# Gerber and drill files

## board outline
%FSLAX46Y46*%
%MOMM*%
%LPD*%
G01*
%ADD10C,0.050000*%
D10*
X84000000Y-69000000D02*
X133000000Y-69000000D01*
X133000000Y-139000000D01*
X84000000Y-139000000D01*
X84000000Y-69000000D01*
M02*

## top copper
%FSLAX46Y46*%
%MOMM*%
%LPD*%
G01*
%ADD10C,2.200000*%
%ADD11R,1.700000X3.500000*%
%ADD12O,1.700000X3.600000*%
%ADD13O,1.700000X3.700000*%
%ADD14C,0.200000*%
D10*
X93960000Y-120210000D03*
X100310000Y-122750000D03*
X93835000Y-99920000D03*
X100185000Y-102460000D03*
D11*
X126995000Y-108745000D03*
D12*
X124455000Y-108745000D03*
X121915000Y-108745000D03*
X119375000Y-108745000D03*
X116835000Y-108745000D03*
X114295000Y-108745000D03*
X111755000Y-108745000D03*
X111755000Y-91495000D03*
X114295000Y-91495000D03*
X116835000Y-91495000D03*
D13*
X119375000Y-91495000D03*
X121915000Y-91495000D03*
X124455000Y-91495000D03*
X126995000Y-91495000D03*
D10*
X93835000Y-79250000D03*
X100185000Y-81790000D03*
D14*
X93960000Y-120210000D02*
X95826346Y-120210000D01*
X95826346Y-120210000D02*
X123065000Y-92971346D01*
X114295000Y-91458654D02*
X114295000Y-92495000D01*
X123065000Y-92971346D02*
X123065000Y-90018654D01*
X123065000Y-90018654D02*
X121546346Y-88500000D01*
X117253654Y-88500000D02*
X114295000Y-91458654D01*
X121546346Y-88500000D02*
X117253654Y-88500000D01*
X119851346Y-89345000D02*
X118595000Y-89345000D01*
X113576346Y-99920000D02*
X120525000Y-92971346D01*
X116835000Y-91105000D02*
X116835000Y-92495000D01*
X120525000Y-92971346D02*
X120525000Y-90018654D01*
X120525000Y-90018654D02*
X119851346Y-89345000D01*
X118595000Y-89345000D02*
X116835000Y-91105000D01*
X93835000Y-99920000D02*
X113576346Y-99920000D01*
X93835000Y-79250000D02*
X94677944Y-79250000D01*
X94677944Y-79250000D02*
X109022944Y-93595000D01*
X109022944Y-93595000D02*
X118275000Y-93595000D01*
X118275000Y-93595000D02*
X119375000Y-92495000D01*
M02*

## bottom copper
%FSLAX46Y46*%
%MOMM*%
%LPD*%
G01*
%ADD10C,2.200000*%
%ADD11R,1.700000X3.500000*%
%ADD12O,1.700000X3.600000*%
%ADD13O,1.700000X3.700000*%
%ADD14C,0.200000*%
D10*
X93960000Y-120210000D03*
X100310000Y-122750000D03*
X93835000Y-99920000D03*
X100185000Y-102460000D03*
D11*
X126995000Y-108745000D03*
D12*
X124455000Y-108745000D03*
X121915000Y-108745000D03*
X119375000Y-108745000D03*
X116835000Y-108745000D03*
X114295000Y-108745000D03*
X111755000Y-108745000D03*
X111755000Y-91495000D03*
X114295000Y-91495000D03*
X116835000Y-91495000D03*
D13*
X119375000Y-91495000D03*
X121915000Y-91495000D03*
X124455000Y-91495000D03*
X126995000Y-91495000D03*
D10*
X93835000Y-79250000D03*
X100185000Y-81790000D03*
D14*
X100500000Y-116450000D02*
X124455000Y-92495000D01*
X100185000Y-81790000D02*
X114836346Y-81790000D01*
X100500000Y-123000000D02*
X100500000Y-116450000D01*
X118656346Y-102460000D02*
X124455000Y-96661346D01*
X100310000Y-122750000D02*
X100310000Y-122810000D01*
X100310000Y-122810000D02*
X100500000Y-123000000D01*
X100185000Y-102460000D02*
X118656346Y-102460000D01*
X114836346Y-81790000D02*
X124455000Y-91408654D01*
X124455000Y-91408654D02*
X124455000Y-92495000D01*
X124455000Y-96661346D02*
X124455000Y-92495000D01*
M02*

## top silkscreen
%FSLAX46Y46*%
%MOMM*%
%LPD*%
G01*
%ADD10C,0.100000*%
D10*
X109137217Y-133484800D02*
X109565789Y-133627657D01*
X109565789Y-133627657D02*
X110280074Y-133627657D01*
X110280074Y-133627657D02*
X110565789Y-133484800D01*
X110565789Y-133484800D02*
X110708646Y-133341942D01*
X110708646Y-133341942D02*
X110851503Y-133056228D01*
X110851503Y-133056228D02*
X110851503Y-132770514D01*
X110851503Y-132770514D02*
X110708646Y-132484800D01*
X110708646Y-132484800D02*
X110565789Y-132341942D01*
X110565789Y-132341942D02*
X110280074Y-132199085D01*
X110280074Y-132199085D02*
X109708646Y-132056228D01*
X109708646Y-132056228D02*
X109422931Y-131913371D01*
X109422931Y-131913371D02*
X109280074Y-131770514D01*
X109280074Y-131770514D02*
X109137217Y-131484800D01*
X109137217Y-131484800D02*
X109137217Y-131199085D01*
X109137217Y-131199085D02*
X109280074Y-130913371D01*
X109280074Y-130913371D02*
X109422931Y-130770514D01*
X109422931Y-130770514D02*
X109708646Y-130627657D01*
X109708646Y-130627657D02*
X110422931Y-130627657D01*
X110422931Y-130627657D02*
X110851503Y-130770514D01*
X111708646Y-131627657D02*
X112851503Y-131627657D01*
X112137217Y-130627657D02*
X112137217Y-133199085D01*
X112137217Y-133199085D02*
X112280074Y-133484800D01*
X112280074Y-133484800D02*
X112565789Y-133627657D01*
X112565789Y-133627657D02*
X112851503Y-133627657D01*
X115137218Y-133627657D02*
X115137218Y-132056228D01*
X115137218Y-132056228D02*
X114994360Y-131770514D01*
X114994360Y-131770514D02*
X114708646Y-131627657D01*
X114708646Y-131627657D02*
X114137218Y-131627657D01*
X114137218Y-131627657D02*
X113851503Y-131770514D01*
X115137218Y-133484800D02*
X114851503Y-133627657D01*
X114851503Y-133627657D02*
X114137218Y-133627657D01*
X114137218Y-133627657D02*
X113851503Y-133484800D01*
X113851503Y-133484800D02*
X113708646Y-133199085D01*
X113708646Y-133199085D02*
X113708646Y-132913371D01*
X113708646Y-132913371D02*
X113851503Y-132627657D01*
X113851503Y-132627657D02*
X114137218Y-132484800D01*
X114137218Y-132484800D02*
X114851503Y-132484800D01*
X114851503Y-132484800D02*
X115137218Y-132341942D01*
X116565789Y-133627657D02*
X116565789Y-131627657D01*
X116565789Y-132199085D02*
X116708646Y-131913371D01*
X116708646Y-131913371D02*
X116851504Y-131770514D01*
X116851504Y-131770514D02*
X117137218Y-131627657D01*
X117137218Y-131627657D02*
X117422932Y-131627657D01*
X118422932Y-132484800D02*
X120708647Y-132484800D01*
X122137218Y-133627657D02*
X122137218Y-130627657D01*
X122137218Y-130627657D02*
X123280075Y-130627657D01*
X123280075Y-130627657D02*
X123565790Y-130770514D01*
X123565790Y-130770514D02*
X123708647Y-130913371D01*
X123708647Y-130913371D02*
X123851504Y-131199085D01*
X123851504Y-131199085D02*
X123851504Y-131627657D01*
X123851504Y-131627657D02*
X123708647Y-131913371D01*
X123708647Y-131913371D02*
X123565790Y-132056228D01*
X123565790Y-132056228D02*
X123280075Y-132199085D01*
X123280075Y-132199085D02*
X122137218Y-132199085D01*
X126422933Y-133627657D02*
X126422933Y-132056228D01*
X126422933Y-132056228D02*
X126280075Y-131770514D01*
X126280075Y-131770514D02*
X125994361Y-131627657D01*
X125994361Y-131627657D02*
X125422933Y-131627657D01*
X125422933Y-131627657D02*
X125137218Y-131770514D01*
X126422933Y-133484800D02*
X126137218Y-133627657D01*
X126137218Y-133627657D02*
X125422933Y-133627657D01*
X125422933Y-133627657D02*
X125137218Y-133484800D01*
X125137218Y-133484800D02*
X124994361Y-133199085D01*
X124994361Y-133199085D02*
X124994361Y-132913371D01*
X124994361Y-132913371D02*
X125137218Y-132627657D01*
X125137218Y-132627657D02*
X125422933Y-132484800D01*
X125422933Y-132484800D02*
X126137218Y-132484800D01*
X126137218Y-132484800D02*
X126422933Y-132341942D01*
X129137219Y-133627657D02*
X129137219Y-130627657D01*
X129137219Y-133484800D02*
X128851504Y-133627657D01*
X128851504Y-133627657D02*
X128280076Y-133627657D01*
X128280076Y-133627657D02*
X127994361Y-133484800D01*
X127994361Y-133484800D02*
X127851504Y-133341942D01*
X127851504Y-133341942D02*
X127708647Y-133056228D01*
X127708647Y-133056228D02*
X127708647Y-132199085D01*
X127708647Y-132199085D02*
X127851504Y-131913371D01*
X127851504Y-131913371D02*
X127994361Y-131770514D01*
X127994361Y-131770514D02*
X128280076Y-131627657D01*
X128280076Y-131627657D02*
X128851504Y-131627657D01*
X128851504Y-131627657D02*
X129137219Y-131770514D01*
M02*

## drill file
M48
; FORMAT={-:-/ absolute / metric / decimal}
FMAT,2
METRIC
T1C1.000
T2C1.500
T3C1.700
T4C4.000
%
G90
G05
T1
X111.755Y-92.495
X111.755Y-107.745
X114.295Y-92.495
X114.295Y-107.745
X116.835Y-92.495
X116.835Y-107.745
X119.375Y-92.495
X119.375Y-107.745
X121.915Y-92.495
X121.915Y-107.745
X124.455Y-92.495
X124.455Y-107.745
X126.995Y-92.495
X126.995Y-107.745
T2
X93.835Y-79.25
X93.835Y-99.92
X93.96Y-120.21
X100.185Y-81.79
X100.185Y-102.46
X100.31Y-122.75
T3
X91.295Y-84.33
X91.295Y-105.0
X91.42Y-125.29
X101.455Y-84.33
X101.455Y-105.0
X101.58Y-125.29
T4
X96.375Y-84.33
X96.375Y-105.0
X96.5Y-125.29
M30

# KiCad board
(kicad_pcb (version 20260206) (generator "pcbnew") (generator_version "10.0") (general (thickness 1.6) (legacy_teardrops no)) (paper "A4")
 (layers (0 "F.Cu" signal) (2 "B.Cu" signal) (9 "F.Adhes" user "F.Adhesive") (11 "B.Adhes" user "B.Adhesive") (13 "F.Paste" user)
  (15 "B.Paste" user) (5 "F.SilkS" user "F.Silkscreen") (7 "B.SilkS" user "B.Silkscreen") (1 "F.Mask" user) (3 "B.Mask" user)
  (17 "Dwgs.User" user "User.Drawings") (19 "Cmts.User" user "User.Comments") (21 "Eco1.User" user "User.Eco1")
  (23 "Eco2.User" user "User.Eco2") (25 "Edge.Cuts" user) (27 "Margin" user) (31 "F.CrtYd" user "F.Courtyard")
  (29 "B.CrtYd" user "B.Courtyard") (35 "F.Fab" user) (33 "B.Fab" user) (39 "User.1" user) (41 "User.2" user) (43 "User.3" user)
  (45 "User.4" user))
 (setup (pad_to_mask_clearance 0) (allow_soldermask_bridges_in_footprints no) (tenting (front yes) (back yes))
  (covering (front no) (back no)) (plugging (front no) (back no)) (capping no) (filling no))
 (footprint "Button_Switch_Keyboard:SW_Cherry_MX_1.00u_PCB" (layer "B.Cu") (at 93.96 120.21 180)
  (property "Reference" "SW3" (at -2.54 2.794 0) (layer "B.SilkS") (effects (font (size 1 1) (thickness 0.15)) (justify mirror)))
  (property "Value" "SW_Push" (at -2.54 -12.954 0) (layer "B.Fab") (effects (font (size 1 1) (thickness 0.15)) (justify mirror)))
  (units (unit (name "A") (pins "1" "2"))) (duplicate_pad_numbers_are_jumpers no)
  (pad "" np_thru_hole circle (at -7.62 -5.08 180) (size 1.7 1.7) (drill 1.7) (layers "*.Cu" "*.Mask"))
  (pad "" np_thru_hole circle (at -2.54 -5.08 180) (size 4 4) (drill 4) (layers "*.Cu" "*.Mask"))
  (pad "" np_thru_hole circle (at 2.54 -5.08 180) (size 1.7 1.7) (drill 1.7) (layers "*.Cu" "*.Mask"))
  (pad "1" thru_hole circle (at 0 0 180) (size 2.2 2.2) (drill 1.5) (layers "*.Cu" "*.Mask") (remove_unused_layers no)
   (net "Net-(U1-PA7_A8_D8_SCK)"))
  (pad "2" thru_hole circle (at -6.35 -2.54 180) (size 2.2 2.2) (drill 1.5) (layers "*.Cu" "*.Mask") (remove_unused_layers no) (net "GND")))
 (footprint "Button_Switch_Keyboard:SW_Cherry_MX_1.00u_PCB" (layer "B.Cu") (at 93.835 99.92 180)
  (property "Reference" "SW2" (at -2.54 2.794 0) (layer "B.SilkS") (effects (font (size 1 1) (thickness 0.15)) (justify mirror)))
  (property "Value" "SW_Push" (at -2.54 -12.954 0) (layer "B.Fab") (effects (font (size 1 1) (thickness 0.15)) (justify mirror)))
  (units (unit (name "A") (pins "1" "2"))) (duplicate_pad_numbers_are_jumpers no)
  (pad "" np_thru_hole circle (at -7.62 -5.08 180) (size 1.7 1.7) (drill 1.7) (layers "*.Cu" "*.Mask"))
  (pad "" np_thru_hole circle (at -2.54 -5.08 180) (size 4 4) (drill 4) (layers "*.Cu" "*.Mask"))
  (pad "" np_thru_hole circle (at 2.54 -5.08 180) (size 1.7 1.7) (drill 1.7) (layers "*.Cu" "*.Mask"))
  (pad "1" thru_hole circle (at 0 0 180) (size 2.2 2.2) (drill 1.5) (layers "*.Cu" "*.Mask") (remove_unused_layers no)
   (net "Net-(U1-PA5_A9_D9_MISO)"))
  (pad "2" thru_hole circle (at -6.35 -2.54 180) (size 2.2 2.2) (drill 1.5) (layers "*.Cu" "*.Mask") (remove_unused_layers no) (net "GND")))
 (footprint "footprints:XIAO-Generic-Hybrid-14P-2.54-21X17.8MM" (layer "B.Cu") (at 119.375 100.12 90)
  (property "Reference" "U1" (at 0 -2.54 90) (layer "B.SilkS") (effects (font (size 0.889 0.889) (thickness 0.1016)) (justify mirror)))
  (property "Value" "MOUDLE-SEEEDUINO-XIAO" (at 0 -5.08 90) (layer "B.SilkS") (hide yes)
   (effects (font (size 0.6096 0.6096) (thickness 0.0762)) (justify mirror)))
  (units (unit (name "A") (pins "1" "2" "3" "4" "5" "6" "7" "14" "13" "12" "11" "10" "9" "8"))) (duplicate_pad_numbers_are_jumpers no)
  (pad "1" thru_hole rect (at -7.625 7.62 90) (size 3.5 1.7) (drill 1 (offset -1 0)) (layers "*.Cu" "*.Mask") (remove_unused_layers no)
   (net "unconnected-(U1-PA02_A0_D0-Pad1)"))
  (pad "2" thru_hole oval (at -7.625 5.08 90) (size 3.6 1.7) (drill 1 (offset -1 0)) (layers "*.Cu" "*.Mask") (remove_unused_layers no)
   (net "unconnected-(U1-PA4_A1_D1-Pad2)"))
  (pad "3" thru_hole oval (at -7.625 2.54 90) (size 3.6 1.7) (drill 1 (offset -1 0)) (layers "*.Cu" "*.Mask") (remove_unused_layers no)
   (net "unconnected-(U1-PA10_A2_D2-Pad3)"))
  (pad "4" thru_hole oval (at -7.625 0 90) (size 3.6 1.7) (drill 1 (offset -1 0)) (layers "*.Cu" "*.Mask") (remove_unused_layers no)
   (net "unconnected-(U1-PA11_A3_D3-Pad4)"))
  (pad "5" thru_hole oval (at -7.625 -2.54 90) (size 3.6 1.7) (drill 1 (offset -1 0)) (layers "*.Cu" "*.Mask") (remove_unused_layers no)
   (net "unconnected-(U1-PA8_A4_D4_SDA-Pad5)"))
  (pad "6" thru_hole oval (at -7.625 -5.08 270) (size 3.6 1.7) (drill 1 (offset 1 0)) (layers "*.Cu" "*.Mask") (remove_unused_layers no)
   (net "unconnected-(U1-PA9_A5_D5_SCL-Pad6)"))
  (pad "7" thru_hole oval (at -7.625 -7.62 90) (size 3.6 1.7) (drill 1 (offset -1 0)) (layers "*.Cu" "*.Mask") (remove_unused_layers no)
   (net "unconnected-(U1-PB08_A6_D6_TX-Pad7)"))
  (pad "8" thru_hole oval (at 7.625 -7.62 90) (size 3.6 1.7) (drill 1 (offset 1 0)) (layers "*.Cu" "*.Mask") (remove_unused_layers no)
   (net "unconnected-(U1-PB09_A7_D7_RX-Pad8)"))
  (pad "9" thru_hole oval (at 7.625 -5.08 90) (size 3.6 1.7) (drill 1 (offset 1 0)) (layers "*.Cu" "*.Mask") (remove_unused_layers no)
   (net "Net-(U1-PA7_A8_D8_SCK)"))
  (pad "10" thru_hole oval (at 7.625 -2.54 90) (size 3.6 1.7) (drill 1 (offset 1 0)) (layers "*.Cu" "*.Mask") (remove_unused_layers no)
   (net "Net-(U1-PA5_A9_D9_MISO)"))
  (pad "11" thru_hole oval (at 7.625 0 90) (size 3.7 1.7) (drill 1 (offset 1 0)) (layers "*.Cu" "*.Mask") (remove_unused_layers no)
   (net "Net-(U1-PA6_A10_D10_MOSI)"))
  (pad "12" thru_hole oval (at 7.625 2.54 90) (size 3.7 1.7) (drill 1 (offset 1 0)) (layers "*.Cu" "*.Mask") (remove_unused_layers no)
   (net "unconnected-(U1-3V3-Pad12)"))
  (pad "13" thru_hole oval (at 7.625 5.08 90) (size 3.7 1.7) (drill 1 (offset 1 0)) (layers "*.Cu" "*.Mask") (remove_unused_layers no)
   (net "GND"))
  (pad "14" thru_hole oval (at 7.625 7.62 90) (size 3.7 1.7) (drill 1 (offset 1 0)) (layers "*.Cu" "*.Mask") (remove_unused_layers no)
   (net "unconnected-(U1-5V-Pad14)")))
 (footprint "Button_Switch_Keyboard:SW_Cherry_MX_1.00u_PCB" (layer "B.Cu") (at 93.835 79.25 180)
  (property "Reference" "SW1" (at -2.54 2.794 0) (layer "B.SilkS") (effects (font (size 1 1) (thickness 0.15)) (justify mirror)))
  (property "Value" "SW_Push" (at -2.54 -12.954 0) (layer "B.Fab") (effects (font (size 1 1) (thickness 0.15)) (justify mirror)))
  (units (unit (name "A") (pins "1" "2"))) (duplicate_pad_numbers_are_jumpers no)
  (pad "" np_thru_hole circle (at -7.62 -5.08 180) (size 1.7 1.7) (drill 1.7) (layers "*.Cu" "*.Mask"))
  (pad "" np_thru_hole circle (at -2.54 -5.08 180) (size 4 4) (drill 4) (layers "*.Cu" "*.Mask"))
  (pad "" np_thru_hole circle (at 2.54 -5.08 180) (size 1.7 1.7) (drill 1.7) (layers "*.Cu" "*.Mask"))
  (pad "1" thru_hole circle (at 0 0 180) (size 2.2 2.2) (drill 1.5) (layers "*.Cu" "*.Mask") (remove_unused_layers no)
   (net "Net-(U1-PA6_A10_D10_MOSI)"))
  (pad "2" thru_hole circle (at -6.35 -2.54 180) (size 2.2 2.2) (drill 1.5) (layers "*.Cu" "*.Mask") (remove_unused_layers no) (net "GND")))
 (gr_rect (start 84 69) (end 133 139) (stroke (width 0.05) (type default)) (fill no) (layer "Edge.Cuts"))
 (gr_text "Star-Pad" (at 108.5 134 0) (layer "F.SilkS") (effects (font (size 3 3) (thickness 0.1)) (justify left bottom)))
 (segment (start 93.96 120.21) (end 95.826346 120.21) (width 0.2) (layer "F.Cu") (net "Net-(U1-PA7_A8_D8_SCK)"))
 (segment (start 95.826346 120.21) (end 123.065 92.971346) (width 0.2) (layer "F.Cu") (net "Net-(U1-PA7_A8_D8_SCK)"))
 (segment (start 114.295 91.458654) (end 114.295 92.495) (width 0.2) (layer "F.Cu") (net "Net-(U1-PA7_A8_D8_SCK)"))
 (segment (start 123.065 92.971346) (end 123.065 90.018654) (width 0.2) (layer "F.Cu") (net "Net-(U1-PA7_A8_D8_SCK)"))
 (segment (start 123.065 90.018654) (end 121.546346 88.5) (width 0.2) (layer "F.Cu") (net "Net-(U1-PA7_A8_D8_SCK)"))
 (segment (start 117.253654 88.5) (end 114.295 91.458654) (width 0.2) (layer "F.Cu") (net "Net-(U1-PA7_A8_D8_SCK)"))
 (segment (start 121.546346 88.5) (end 117.253654 88.5) (width 0.2) (layer "F.Cu") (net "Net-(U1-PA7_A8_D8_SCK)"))
 (segment (start 100.5 116.45) (end 124.455 92.495) (width 0.2) (layer "B.Cu") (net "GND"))
 (segment (start 100.185 81.79) (end 114.836346 81.79) (width 0.2) (layer "B.Cu") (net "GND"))
 (segment (start 100.5 123) (end 100.5 116.45) (width 0.2) (layer "B.Cu") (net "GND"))
 (segment (start 118.656346 102.46) (end 124.455 96.661346) (width 0.2) (layer "B.Cu") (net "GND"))
 (segment (start 100.31 122.75) (end 100.31 122.81) (width 0.2) (layer "B.Cu") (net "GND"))
 (segment (start 100.31 122.81) (end 100.5 123) (width 0.2) (layer "B.Cu") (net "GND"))
 (segment (start 100.185 102.46) (end 118.656346 102.46) (width 0.2) (layer "B.Cu") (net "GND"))
 (segment (start 114.836346 81.79) (end 124.455 91.408654) (width 0.2) (layer "B.Cu") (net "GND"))
 (segment (start 124.455 91.408654) (end 124.455 92.495) (width 0.2) (layer "B.Cu") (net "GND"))
 (segment (start 124.455 96.661346) (end 124.455 92.495) (width 0.2) (layer "B.Cu") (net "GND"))
 (segment (start 119.851346 89.345) (end 118.595 89.345) (width 0.2) (layer "F.Cu") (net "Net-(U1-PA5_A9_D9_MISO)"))
 (segment (start 113.576346 99.92) (end 120.525 92.971346) (width 0.2) (layer "F.Cu") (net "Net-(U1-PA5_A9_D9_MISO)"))
 (segment (start 116.835 91.105) (end 116.835 92.495) (width 0.2) (layer "F.Cu") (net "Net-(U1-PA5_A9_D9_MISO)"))
 (segment (start 120.525 92.971346) (end 120.525 90.018654) (width 0.2) (layer "F.Cu") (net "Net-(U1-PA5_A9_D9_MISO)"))
 (segment (start 120.525 90.018654) (end 119.851346 89.345) (width 0.2) (layer "F.Cu") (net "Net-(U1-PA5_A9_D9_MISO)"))
 (segment (start 118.595 89.345) (end 116.835 91.105) (width 0.2) (layer "F.Cu") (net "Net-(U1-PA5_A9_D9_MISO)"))
 (segment (start 93.835 99.92) (end 113.576346 99.92) (width 0.2) (layer "F.Cu") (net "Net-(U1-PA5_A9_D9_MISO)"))
 (segment (start 93.835 79.25) (end 94.677944 79.25) (width 0.2) (layer "F.Cu") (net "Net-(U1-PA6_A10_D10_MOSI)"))
 (segment (start 94.677944 79.25) (end 109.022944 93.595) (width 0.2) (layer "F.Cu") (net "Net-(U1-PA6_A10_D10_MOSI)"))
 (segment (start 109.022944 93.595) (end 118.275 93.595) (width 0.2) (layer "F.Cu") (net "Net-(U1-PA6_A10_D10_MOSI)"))
 (segment (start 118.275 93.595) (end 119.375 92.495) (width 0.2) (layer "F.Cu") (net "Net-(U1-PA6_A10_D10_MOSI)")))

